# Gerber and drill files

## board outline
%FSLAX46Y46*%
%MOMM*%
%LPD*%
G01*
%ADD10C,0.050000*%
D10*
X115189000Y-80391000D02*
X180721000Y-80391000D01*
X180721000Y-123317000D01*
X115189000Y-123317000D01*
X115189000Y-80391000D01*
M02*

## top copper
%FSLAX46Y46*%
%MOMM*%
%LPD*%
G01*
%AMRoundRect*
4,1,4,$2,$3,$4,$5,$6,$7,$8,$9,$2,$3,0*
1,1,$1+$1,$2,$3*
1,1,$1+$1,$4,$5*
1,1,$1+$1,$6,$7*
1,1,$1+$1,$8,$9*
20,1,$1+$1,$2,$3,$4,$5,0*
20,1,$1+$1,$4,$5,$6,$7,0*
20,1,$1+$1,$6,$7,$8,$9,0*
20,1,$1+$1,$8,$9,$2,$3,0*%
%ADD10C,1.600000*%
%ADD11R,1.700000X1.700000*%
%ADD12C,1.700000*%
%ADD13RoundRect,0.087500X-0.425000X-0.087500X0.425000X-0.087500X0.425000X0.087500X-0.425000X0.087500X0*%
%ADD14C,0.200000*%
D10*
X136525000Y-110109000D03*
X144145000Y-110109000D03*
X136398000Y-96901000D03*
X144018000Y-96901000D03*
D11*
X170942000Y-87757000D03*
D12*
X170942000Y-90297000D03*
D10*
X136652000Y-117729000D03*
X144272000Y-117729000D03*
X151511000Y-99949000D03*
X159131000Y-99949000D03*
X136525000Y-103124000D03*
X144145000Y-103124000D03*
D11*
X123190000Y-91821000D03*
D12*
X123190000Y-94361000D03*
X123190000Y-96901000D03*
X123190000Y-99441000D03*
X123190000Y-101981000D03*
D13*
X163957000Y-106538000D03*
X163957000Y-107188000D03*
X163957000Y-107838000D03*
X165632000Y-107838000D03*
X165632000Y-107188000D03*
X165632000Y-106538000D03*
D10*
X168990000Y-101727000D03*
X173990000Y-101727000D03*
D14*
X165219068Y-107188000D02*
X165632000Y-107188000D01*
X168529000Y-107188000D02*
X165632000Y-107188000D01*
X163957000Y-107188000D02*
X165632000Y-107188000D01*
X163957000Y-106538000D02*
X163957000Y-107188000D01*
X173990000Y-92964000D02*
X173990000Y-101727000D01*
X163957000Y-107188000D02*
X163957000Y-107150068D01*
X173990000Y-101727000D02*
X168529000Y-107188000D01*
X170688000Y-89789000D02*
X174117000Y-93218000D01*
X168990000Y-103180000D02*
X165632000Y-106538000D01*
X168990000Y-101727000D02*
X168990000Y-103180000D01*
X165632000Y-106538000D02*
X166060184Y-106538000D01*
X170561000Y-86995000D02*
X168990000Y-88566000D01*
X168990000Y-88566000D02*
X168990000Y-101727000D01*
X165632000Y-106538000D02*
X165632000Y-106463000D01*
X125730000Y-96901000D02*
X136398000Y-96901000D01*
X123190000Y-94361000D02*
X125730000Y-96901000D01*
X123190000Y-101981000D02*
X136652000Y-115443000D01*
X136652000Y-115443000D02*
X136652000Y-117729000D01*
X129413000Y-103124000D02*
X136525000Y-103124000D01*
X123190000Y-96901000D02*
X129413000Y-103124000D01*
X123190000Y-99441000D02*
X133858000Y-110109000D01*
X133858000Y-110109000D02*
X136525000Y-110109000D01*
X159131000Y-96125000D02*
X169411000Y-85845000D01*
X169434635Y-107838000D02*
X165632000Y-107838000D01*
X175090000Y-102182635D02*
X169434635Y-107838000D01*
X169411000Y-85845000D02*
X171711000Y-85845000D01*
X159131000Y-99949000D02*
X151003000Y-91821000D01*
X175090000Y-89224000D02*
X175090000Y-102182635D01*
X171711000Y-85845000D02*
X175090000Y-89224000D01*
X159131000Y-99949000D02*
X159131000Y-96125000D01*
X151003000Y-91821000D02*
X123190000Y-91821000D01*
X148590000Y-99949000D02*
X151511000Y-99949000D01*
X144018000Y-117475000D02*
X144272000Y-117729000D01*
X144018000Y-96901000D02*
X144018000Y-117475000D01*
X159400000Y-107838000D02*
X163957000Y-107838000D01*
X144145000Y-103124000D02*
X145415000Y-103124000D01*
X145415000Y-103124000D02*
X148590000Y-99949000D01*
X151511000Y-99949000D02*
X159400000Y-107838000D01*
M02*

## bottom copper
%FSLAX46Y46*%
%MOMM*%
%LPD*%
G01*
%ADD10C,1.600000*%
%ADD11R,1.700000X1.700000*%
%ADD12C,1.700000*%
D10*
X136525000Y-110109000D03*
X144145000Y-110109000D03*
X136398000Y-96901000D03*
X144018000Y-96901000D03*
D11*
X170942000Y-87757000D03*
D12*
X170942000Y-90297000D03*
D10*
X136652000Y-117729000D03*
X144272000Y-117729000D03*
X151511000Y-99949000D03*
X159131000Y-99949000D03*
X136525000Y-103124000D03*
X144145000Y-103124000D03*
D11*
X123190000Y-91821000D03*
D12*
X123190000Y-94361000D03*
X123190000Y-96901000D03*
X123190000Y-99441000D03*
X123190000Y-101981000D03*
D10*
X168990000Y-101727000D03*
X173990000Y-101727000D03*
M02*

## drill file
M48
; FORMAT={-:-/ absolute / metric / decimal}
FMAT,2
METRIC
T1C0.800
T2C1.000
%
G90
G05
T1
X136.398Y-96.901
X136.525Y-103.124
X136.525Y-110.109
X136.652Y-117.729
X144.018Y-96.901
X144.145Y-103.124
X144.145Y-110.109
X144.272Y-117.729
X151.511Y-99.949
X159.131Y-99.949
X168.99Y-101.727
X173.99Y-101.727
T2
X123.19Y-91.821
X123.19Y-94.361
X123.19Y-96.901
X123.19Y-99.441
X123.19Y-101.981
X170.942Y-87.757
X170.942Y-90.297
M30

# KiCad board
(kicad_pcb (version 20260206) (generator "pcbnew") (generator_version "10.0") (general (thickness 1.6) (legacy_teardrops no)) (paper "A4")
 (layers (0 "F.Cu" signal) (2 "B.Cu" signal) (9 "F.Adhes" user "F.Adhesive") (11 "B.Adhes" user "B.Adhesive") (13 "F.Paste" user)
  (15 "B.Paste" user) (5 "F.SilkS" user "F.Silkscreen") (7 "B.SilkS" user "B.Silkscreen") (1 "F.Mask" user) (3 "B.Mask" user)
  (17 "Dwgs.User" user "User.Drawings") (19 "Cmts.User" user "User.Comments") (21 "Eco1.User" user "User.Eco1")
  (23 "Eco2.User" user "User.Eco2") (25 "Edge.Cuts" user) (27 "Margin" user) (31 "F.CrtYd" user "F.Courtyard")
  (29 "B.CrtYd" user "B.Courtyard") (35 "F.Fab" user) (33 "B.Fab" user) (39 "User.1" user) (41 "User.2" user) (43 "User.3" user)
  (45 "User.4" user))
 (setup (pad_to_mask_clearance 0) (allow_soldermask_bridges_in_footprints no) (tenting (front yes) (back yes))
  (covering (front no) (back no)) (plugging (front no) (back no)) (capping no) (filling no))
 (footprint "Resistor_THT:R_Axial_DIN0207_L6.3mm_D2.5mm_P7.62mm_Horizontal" (layer "F.Cu") (at 136.525 110.109)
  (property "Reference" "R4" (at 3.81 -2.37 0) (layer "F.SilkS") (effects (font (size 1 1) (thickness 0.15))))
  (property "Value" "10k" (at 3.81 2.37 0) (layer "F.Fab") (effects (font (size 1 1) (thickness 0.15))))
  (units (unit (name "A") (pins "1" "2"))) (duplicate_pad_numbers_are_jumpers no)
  (pad "1" thru_hole circle (at 0 0) (size 1.6 1.6) (drill 0.8) (layers "*.Cu" "*.Mask") (remove_unused_layers no) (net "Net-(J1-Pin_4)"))
  (pad "2" thru_hole circle (at 7.62 0) (size 1.6 1.6) (drill 0.8) (layers "*.Cu" "*.Mask") (remove_unused_layers no) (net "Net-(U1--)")))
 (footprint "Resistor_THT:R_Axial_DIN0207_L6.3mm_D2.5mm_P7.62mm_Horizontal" (layer "F.Cu") (at 136.398 96.901)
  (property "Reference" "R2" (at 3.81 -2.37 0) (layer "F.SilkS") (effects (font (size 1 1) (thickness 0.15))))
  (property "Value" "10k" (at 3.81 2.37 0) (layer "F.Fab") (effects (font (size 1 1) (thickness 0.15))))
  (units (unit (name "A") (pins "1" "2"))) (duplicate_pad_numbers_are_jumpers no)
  (pad "1" thru_hole circle (at 0 0) (size 1.6 1.6) (drill 0.8) (layers "*.Cu" "*.Mask") (remove_unused_layers no) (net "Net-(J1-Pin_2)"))
  (pad "2" thru_hole circle (at 7.62 0) (size 1.6 1.6) (drill 0.8) (layers "*.Cu" "*.Mask") (remove_unused_layers no) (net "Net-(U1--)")))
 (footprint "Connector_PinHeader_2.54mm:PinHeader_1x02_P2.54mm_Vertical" (layer "F.Cu") (at 170.942 87.757)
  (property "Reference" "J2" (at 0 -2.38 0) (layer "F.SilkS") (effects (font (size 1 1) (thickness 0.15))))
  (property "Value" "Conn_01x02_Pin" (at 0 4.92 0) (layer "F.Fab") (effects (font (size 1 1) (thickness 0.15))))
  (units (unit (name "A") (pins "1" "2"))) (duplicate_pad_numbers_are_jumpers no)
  (pad "1" thru_hole rect (at 0 0) (size 1.7 1.7) (drill 1) (layers "*.Cu" "*.Mask") (remove_unused_layers no) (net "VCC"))
  (pad "2" thru_hole circle (at 0 2.54) (size 1.7 1.7) (drill 1) (layers "*.Cu" "*.Mask") (remove_unused_layers no) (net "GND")))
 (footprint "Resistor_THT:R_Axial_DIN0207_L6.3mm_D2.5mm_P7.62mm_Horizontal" (layer "F.Cu") (at 136.652 117.729)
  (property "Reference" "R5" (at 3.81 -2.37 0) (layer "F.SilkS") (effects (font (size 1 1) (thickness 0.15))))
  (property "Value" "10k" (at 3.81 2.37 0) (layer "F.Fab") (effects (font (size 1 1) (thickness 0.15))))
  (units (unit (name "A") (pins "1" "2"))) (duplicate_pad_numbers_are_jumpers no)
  (pad "1" thru_hole circle (at 0 0) (size 1.6 1.6) (drill 0.8) (layers "*.Cu" "*.Mask") (remove_unused_layers no) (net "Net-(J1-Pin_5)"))
  (pad "2" thru_hole circle (at 7.62 0) (size 1.6 1.6) (drill 0.8) (layers "*.Cu" "*.Mask") (remove_unused_layers no) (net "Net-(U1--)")))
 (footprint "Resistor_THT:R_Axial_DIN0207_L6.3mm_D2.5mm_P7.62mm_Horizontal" (layer "F.Cu") (at 151.511 99.949)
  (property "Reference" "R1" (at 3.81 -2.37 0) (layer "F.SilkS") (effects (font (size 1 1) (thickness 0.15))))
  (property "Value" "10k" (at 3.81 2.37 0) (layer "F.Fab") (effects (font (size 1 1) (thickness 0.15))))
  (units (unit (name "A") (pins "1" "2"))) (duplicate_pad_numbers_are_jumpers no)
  (pad "1" thru_hole circle (at 0 0) (size 1.6 1.6) (drill 0.8) (layers "*.Cu" "*.Mask") (remove_unused_layers no) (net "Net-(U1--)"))
  (pad "2" thru_hole circle (at 7.62 0) (size 1.6 1.6) (drill 0.8) (layers "*.Cu" "*.Mask") (remove_unused_layers no) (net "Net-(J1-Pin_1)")))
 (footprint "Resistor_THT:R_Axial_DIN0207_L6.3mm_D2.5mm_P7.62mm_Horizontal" (layer "F.Cu") (at 136.525 103.124)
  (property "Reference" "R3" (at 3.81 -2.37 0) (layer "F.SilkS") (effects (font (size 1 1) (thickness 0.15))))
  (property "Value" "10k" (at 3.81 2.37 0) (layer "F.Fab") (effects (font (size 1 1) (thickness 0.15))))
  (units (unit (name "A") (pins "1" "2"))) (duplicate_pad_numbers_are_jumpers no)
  (pad "1" thru_hole circle (at 0 0) (size 1.6 1.6) (drill 0.8) (layers "*.Cu" "*.Mask") (remove_unused_layers no) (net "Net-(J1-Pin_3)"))
  (pad "2" thru_hole circle (at 7.62 0) (size 1.6 1.6) (drill 0.8) (layers "*.Cu" "*.Mask") (remove_unused_layers no) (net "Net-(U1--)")))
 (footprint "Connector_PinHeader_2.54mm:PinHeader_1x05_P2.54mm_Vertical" (layer "F.Cu") (at 123.19 91.821)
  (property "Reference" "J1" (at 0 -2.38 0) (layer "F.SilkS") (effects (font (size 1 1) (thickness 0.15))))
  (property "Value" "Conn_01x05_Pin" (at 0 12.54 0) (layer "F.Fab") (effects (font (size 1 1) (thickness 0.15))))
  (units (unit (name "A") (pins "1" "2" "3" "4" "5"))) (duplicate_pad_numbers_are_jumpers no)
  (pad "1" thru_hole rect (at 0 0) (size 1.7 1.7) (drill 1) (layers "*.Cu" "*.Mask") (remove_unused_layers no) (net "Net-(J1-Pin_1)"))
  (pad "2" thru_hole circle (at 0 2.54) (size 1.7 1.7) (drill 1) (layers "*.Cu" "*.Mask") (remove_unused_layers no) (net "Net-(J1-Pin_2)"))
  (pad "3" thru_hole circle (at 0 5.08) (size 1.7 1.7) (drill 1) (layers "*.Cu" "*.Mask") (remove_unused_layers no) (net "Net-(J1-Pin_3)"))
  (pad "4" thru_hole circle (at 0 7.62) (size 1.7 1.7) (drill 1) (layers "*.Cu" "*.Mask") (remove_unused_layers no) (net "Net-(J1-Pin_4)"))
  (pad "5" thru_hole circle (at 0 10.16) (size 1.7 1.7) (drill 1) (layers "*.Cu" "*.Mask") (remove_unused_layers no) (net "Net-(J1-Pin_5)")))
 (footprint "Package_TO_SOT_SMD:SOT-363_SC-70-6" (layer "F.Cu") (at 164.7945 107.188)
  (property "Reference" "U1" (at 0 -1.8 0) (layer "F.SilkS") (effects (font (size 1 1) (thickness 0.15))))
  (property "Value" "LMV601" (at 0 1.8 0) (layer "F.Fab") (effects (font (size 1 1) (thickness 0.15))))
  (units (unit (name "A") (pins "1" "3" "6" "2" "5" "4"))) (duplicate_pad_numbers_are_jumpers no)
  (pad "1" smd roundrect (at -0.8375 -0.65) (size 1.025 0.35) (layers "F.Cu" "F.Mask" "F.Paste") (roundrect_rratio 0.25) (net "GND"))
  (pad "2" smd roundrect (at -0.8375 0) (size 1.025 0.35) (layers "F.Cu" "F.Mask" "F.Paste") (roundrect_rratio 0.25) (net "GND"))
  (pad "3" smd roundrect (at -0.8375 0.65) (size 1.025 0.35) (layers "F.Cu" "F.Mask" "F.Paste") (roundrect_rratio 0.25) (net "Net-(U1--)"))
  (pad "4" smd roundrect (at 0.8375 0.65) (size 1.025 0.35) (layers "F.Cu" "F.Mask" "F.Paste") (roundrect_rratio 0.25)
   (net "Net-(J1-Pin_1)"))
  (pad "5" smd roundrect (at 0.8375 0) (size 1.025 0.35) (layers "F.Cu" "F.Mask" "F.Paste") (roundrect_rratio 0.25) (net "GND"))
  (pad "6" smd roundrect (at 0.8375 -0.65) (size 1.025 0.35) (layers "F.Cu" "F.Mask" "F.Paste") (roundrect_rratio 0.25) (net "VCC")))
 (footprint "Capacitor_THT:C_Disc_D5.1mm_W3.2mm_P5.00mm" (layer "F.Cu") (at 168.99 101.727)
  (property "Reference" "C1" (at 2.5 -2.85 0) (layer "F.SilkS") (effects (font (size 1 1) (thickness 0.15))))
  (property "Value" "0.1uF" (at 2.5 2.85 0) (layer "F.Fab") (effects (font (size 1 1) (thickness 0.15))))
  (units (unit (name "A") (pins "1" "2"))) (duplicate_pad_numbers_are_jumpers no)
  (pad "1" thru_hole circle (at 0 0) (size 1.6 1.6) (drill 0.8) (layers "*.Cu" "*.Mask") (remove_unused_layers no) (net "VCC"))
  (pad "2" thru_hole circle (at 5 0) (size 1.6 1.6) (drill 0.8) (layers "*.Cu" "*.Mask") (remove_unused_layers no) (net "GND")))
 (gr_rect (start 115.189 80.391) (end 180.721 123.317) (stroke (width 0.05) (type default)) (fill no) (layer "Edge.Cuts"))
 (segment (start 165.219068 107.188) (end 165.632 107.188) (width 0.2) (layer "F.Cu") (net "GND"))
 (segment (start 168.529 107.188) (end 165.632 107.188) (width 0.2) (layer "F.Cu") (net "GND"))
 (segment (start 163.957 107.188) (end 165.632 107.188) (width 0.2) (layer "F.Cu") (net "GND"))
 (segment (start 163.957 106.538) (end 163.957 107.188) (width 0.2) (layer "F.Cu") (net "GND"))
 (segment (start 173.99 92.964) (end 173.99 101.727) (width 0.2) (layer "F.Cu") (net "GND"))
 (segment (start 163.957 107.188) (end 163.957 107.150068) (width 0.2) (layer "F.Cu") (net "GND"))
 (segment (start 173.99 101.727) (end 168.529 107.188) (width 0.2) (layer "F.Cu") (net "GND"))
 (segment (start 170.688 89.789) (end 174.117 93.218) (width 0.2) (layer "F.Cu") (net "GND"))
 (segment (start 168.99 103.18) (end 165.632 106.538) (width 0.2) (layer "F.Cu") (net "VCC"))
 (segment (start 168.99 101.727) (end 168.99 103.18) (width 0.2) (layer "F.Cu") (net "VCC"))
 (segment (start 165.632 106.538) (end 166.060184 106.538) (width 0.2) (layer "F.Cu") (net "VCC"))
 (segment (start 170.561 86.995) (end 168.99 88.566) (width 0.2) (layer "F.Cu") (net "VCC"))
 (segment (start 168.99 88.566) (end 168.99 101.727) (width 0.2) (layer "F.Cu") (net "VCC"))
 (segment (start 165.632 106.538) (end 165.632 106.463) (width 0.2) (layer "F.Cu") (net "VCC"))
 (segment (start 125.73 96.901) (end 136.398 96.901) (width 0.2) (layer "F.Cu") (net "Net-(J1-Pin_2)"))
 (segment (start 123.19 94.361) (end 125.73 96.901) (width 0.2) (layer "F.Cu") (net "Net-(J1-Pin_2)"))
 (segment (start 123.19 101.981) (end 136.652 115.443) (width 0.2) (layer "F.Cu") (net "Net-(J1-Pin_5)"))
 (segment (start 136.652 115.443) (end 136.652 117.729) (width 0.2) (layer "F.Cu") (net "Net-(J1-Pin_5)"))
 (segment (start 129.413 103.124) (end 136.525 103.124) (width 0.2) (layer "F.Cu") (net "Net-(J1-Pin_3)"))
 (segment (start 123.19 96.901) (end 129.413 103.124) (width 0.2) (layer "F.Cu") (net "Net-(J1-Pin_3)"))
 (segment (start 123.19 99.441) (end 133.858 110.109) (width 0.2) (layer "F.Cu") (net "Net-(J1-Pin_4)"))
 (segment (start 133.858 110.109) (end 136.525 110.109) (width 0.2) (layer "F.Cu") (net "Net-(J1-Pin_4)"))
 (segment (start 159.131 96.125) (end 169.411 85.845) (width 0.2) (layer "F.Cu") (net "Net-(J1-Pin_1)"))
 (segment (start 169.434635 107.838) (end 165.632 107.838) (width 0.2) (layer "F.Cu") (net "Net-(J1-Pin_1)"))
 (segment (start 175.09 102.182635) (end 169.434635 107.838) (width 0.2) (layer "F.Cu") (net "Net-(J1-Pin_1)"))
 (segment (start 169.411 85.845) (end 171.711 85.845) (width 0.2) (layer "F.Cu") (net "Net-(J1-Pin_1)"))
 (segment (start 159.131 99.949) (end 151.003 91.821) (width 0.2) (layer "F.Cu") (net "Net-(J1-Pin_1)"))
 (segment (start 175.09 89.224) (end 175.09 102.182635) (width 0.2) (layer "F.Cu") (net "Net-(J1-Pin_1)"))
 (segment (start 171.711 85.845) (end 175.09 89.224) (width 0.2) (layer "F.Cu") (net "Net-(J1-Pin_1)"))
 (segment (start 159.131 99.949) (end 159.131 96.125) (width 0.2) (layer "F.Cu") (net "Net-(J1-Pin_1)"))
 (segment (start 151.003 91.821) (end 123.19 91.821) (width 0.2) (layer "F.Cu") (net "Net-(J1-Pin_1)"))
 (segment (start 148.59 99.949) (end 151.511 99.949) (width 0.2) (layer "F.Cu") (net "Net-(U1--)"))
 (segment (start 144.018 117.475) (end 144.272 117.729) (width 0.2) (layer "F.Cu") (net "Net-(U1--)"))
 (segment (start 144.018 96.901) (end 144.018 117.475) (width 0.2) (layer "F.Cu") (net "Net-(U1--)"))
 (segment (start 159.4 107.838) (end 163.957 107.838) (width 0.2) (layer "F.Cu") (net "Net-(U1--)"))
 (segment (start 144.145 103.124) (end 145.415 103.124) (width 0.2) (layer "F.Cu") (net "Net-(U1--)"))
 (segment (start 145.415 103.124) (end 148.59 99.949) (width 0.2) (layer "F.Cu") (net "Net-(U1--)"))
 (segment (start 151.511 99.949) (end 159.4 107.838) (width 0.2) (layer "F.Cu") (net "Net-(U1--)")))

